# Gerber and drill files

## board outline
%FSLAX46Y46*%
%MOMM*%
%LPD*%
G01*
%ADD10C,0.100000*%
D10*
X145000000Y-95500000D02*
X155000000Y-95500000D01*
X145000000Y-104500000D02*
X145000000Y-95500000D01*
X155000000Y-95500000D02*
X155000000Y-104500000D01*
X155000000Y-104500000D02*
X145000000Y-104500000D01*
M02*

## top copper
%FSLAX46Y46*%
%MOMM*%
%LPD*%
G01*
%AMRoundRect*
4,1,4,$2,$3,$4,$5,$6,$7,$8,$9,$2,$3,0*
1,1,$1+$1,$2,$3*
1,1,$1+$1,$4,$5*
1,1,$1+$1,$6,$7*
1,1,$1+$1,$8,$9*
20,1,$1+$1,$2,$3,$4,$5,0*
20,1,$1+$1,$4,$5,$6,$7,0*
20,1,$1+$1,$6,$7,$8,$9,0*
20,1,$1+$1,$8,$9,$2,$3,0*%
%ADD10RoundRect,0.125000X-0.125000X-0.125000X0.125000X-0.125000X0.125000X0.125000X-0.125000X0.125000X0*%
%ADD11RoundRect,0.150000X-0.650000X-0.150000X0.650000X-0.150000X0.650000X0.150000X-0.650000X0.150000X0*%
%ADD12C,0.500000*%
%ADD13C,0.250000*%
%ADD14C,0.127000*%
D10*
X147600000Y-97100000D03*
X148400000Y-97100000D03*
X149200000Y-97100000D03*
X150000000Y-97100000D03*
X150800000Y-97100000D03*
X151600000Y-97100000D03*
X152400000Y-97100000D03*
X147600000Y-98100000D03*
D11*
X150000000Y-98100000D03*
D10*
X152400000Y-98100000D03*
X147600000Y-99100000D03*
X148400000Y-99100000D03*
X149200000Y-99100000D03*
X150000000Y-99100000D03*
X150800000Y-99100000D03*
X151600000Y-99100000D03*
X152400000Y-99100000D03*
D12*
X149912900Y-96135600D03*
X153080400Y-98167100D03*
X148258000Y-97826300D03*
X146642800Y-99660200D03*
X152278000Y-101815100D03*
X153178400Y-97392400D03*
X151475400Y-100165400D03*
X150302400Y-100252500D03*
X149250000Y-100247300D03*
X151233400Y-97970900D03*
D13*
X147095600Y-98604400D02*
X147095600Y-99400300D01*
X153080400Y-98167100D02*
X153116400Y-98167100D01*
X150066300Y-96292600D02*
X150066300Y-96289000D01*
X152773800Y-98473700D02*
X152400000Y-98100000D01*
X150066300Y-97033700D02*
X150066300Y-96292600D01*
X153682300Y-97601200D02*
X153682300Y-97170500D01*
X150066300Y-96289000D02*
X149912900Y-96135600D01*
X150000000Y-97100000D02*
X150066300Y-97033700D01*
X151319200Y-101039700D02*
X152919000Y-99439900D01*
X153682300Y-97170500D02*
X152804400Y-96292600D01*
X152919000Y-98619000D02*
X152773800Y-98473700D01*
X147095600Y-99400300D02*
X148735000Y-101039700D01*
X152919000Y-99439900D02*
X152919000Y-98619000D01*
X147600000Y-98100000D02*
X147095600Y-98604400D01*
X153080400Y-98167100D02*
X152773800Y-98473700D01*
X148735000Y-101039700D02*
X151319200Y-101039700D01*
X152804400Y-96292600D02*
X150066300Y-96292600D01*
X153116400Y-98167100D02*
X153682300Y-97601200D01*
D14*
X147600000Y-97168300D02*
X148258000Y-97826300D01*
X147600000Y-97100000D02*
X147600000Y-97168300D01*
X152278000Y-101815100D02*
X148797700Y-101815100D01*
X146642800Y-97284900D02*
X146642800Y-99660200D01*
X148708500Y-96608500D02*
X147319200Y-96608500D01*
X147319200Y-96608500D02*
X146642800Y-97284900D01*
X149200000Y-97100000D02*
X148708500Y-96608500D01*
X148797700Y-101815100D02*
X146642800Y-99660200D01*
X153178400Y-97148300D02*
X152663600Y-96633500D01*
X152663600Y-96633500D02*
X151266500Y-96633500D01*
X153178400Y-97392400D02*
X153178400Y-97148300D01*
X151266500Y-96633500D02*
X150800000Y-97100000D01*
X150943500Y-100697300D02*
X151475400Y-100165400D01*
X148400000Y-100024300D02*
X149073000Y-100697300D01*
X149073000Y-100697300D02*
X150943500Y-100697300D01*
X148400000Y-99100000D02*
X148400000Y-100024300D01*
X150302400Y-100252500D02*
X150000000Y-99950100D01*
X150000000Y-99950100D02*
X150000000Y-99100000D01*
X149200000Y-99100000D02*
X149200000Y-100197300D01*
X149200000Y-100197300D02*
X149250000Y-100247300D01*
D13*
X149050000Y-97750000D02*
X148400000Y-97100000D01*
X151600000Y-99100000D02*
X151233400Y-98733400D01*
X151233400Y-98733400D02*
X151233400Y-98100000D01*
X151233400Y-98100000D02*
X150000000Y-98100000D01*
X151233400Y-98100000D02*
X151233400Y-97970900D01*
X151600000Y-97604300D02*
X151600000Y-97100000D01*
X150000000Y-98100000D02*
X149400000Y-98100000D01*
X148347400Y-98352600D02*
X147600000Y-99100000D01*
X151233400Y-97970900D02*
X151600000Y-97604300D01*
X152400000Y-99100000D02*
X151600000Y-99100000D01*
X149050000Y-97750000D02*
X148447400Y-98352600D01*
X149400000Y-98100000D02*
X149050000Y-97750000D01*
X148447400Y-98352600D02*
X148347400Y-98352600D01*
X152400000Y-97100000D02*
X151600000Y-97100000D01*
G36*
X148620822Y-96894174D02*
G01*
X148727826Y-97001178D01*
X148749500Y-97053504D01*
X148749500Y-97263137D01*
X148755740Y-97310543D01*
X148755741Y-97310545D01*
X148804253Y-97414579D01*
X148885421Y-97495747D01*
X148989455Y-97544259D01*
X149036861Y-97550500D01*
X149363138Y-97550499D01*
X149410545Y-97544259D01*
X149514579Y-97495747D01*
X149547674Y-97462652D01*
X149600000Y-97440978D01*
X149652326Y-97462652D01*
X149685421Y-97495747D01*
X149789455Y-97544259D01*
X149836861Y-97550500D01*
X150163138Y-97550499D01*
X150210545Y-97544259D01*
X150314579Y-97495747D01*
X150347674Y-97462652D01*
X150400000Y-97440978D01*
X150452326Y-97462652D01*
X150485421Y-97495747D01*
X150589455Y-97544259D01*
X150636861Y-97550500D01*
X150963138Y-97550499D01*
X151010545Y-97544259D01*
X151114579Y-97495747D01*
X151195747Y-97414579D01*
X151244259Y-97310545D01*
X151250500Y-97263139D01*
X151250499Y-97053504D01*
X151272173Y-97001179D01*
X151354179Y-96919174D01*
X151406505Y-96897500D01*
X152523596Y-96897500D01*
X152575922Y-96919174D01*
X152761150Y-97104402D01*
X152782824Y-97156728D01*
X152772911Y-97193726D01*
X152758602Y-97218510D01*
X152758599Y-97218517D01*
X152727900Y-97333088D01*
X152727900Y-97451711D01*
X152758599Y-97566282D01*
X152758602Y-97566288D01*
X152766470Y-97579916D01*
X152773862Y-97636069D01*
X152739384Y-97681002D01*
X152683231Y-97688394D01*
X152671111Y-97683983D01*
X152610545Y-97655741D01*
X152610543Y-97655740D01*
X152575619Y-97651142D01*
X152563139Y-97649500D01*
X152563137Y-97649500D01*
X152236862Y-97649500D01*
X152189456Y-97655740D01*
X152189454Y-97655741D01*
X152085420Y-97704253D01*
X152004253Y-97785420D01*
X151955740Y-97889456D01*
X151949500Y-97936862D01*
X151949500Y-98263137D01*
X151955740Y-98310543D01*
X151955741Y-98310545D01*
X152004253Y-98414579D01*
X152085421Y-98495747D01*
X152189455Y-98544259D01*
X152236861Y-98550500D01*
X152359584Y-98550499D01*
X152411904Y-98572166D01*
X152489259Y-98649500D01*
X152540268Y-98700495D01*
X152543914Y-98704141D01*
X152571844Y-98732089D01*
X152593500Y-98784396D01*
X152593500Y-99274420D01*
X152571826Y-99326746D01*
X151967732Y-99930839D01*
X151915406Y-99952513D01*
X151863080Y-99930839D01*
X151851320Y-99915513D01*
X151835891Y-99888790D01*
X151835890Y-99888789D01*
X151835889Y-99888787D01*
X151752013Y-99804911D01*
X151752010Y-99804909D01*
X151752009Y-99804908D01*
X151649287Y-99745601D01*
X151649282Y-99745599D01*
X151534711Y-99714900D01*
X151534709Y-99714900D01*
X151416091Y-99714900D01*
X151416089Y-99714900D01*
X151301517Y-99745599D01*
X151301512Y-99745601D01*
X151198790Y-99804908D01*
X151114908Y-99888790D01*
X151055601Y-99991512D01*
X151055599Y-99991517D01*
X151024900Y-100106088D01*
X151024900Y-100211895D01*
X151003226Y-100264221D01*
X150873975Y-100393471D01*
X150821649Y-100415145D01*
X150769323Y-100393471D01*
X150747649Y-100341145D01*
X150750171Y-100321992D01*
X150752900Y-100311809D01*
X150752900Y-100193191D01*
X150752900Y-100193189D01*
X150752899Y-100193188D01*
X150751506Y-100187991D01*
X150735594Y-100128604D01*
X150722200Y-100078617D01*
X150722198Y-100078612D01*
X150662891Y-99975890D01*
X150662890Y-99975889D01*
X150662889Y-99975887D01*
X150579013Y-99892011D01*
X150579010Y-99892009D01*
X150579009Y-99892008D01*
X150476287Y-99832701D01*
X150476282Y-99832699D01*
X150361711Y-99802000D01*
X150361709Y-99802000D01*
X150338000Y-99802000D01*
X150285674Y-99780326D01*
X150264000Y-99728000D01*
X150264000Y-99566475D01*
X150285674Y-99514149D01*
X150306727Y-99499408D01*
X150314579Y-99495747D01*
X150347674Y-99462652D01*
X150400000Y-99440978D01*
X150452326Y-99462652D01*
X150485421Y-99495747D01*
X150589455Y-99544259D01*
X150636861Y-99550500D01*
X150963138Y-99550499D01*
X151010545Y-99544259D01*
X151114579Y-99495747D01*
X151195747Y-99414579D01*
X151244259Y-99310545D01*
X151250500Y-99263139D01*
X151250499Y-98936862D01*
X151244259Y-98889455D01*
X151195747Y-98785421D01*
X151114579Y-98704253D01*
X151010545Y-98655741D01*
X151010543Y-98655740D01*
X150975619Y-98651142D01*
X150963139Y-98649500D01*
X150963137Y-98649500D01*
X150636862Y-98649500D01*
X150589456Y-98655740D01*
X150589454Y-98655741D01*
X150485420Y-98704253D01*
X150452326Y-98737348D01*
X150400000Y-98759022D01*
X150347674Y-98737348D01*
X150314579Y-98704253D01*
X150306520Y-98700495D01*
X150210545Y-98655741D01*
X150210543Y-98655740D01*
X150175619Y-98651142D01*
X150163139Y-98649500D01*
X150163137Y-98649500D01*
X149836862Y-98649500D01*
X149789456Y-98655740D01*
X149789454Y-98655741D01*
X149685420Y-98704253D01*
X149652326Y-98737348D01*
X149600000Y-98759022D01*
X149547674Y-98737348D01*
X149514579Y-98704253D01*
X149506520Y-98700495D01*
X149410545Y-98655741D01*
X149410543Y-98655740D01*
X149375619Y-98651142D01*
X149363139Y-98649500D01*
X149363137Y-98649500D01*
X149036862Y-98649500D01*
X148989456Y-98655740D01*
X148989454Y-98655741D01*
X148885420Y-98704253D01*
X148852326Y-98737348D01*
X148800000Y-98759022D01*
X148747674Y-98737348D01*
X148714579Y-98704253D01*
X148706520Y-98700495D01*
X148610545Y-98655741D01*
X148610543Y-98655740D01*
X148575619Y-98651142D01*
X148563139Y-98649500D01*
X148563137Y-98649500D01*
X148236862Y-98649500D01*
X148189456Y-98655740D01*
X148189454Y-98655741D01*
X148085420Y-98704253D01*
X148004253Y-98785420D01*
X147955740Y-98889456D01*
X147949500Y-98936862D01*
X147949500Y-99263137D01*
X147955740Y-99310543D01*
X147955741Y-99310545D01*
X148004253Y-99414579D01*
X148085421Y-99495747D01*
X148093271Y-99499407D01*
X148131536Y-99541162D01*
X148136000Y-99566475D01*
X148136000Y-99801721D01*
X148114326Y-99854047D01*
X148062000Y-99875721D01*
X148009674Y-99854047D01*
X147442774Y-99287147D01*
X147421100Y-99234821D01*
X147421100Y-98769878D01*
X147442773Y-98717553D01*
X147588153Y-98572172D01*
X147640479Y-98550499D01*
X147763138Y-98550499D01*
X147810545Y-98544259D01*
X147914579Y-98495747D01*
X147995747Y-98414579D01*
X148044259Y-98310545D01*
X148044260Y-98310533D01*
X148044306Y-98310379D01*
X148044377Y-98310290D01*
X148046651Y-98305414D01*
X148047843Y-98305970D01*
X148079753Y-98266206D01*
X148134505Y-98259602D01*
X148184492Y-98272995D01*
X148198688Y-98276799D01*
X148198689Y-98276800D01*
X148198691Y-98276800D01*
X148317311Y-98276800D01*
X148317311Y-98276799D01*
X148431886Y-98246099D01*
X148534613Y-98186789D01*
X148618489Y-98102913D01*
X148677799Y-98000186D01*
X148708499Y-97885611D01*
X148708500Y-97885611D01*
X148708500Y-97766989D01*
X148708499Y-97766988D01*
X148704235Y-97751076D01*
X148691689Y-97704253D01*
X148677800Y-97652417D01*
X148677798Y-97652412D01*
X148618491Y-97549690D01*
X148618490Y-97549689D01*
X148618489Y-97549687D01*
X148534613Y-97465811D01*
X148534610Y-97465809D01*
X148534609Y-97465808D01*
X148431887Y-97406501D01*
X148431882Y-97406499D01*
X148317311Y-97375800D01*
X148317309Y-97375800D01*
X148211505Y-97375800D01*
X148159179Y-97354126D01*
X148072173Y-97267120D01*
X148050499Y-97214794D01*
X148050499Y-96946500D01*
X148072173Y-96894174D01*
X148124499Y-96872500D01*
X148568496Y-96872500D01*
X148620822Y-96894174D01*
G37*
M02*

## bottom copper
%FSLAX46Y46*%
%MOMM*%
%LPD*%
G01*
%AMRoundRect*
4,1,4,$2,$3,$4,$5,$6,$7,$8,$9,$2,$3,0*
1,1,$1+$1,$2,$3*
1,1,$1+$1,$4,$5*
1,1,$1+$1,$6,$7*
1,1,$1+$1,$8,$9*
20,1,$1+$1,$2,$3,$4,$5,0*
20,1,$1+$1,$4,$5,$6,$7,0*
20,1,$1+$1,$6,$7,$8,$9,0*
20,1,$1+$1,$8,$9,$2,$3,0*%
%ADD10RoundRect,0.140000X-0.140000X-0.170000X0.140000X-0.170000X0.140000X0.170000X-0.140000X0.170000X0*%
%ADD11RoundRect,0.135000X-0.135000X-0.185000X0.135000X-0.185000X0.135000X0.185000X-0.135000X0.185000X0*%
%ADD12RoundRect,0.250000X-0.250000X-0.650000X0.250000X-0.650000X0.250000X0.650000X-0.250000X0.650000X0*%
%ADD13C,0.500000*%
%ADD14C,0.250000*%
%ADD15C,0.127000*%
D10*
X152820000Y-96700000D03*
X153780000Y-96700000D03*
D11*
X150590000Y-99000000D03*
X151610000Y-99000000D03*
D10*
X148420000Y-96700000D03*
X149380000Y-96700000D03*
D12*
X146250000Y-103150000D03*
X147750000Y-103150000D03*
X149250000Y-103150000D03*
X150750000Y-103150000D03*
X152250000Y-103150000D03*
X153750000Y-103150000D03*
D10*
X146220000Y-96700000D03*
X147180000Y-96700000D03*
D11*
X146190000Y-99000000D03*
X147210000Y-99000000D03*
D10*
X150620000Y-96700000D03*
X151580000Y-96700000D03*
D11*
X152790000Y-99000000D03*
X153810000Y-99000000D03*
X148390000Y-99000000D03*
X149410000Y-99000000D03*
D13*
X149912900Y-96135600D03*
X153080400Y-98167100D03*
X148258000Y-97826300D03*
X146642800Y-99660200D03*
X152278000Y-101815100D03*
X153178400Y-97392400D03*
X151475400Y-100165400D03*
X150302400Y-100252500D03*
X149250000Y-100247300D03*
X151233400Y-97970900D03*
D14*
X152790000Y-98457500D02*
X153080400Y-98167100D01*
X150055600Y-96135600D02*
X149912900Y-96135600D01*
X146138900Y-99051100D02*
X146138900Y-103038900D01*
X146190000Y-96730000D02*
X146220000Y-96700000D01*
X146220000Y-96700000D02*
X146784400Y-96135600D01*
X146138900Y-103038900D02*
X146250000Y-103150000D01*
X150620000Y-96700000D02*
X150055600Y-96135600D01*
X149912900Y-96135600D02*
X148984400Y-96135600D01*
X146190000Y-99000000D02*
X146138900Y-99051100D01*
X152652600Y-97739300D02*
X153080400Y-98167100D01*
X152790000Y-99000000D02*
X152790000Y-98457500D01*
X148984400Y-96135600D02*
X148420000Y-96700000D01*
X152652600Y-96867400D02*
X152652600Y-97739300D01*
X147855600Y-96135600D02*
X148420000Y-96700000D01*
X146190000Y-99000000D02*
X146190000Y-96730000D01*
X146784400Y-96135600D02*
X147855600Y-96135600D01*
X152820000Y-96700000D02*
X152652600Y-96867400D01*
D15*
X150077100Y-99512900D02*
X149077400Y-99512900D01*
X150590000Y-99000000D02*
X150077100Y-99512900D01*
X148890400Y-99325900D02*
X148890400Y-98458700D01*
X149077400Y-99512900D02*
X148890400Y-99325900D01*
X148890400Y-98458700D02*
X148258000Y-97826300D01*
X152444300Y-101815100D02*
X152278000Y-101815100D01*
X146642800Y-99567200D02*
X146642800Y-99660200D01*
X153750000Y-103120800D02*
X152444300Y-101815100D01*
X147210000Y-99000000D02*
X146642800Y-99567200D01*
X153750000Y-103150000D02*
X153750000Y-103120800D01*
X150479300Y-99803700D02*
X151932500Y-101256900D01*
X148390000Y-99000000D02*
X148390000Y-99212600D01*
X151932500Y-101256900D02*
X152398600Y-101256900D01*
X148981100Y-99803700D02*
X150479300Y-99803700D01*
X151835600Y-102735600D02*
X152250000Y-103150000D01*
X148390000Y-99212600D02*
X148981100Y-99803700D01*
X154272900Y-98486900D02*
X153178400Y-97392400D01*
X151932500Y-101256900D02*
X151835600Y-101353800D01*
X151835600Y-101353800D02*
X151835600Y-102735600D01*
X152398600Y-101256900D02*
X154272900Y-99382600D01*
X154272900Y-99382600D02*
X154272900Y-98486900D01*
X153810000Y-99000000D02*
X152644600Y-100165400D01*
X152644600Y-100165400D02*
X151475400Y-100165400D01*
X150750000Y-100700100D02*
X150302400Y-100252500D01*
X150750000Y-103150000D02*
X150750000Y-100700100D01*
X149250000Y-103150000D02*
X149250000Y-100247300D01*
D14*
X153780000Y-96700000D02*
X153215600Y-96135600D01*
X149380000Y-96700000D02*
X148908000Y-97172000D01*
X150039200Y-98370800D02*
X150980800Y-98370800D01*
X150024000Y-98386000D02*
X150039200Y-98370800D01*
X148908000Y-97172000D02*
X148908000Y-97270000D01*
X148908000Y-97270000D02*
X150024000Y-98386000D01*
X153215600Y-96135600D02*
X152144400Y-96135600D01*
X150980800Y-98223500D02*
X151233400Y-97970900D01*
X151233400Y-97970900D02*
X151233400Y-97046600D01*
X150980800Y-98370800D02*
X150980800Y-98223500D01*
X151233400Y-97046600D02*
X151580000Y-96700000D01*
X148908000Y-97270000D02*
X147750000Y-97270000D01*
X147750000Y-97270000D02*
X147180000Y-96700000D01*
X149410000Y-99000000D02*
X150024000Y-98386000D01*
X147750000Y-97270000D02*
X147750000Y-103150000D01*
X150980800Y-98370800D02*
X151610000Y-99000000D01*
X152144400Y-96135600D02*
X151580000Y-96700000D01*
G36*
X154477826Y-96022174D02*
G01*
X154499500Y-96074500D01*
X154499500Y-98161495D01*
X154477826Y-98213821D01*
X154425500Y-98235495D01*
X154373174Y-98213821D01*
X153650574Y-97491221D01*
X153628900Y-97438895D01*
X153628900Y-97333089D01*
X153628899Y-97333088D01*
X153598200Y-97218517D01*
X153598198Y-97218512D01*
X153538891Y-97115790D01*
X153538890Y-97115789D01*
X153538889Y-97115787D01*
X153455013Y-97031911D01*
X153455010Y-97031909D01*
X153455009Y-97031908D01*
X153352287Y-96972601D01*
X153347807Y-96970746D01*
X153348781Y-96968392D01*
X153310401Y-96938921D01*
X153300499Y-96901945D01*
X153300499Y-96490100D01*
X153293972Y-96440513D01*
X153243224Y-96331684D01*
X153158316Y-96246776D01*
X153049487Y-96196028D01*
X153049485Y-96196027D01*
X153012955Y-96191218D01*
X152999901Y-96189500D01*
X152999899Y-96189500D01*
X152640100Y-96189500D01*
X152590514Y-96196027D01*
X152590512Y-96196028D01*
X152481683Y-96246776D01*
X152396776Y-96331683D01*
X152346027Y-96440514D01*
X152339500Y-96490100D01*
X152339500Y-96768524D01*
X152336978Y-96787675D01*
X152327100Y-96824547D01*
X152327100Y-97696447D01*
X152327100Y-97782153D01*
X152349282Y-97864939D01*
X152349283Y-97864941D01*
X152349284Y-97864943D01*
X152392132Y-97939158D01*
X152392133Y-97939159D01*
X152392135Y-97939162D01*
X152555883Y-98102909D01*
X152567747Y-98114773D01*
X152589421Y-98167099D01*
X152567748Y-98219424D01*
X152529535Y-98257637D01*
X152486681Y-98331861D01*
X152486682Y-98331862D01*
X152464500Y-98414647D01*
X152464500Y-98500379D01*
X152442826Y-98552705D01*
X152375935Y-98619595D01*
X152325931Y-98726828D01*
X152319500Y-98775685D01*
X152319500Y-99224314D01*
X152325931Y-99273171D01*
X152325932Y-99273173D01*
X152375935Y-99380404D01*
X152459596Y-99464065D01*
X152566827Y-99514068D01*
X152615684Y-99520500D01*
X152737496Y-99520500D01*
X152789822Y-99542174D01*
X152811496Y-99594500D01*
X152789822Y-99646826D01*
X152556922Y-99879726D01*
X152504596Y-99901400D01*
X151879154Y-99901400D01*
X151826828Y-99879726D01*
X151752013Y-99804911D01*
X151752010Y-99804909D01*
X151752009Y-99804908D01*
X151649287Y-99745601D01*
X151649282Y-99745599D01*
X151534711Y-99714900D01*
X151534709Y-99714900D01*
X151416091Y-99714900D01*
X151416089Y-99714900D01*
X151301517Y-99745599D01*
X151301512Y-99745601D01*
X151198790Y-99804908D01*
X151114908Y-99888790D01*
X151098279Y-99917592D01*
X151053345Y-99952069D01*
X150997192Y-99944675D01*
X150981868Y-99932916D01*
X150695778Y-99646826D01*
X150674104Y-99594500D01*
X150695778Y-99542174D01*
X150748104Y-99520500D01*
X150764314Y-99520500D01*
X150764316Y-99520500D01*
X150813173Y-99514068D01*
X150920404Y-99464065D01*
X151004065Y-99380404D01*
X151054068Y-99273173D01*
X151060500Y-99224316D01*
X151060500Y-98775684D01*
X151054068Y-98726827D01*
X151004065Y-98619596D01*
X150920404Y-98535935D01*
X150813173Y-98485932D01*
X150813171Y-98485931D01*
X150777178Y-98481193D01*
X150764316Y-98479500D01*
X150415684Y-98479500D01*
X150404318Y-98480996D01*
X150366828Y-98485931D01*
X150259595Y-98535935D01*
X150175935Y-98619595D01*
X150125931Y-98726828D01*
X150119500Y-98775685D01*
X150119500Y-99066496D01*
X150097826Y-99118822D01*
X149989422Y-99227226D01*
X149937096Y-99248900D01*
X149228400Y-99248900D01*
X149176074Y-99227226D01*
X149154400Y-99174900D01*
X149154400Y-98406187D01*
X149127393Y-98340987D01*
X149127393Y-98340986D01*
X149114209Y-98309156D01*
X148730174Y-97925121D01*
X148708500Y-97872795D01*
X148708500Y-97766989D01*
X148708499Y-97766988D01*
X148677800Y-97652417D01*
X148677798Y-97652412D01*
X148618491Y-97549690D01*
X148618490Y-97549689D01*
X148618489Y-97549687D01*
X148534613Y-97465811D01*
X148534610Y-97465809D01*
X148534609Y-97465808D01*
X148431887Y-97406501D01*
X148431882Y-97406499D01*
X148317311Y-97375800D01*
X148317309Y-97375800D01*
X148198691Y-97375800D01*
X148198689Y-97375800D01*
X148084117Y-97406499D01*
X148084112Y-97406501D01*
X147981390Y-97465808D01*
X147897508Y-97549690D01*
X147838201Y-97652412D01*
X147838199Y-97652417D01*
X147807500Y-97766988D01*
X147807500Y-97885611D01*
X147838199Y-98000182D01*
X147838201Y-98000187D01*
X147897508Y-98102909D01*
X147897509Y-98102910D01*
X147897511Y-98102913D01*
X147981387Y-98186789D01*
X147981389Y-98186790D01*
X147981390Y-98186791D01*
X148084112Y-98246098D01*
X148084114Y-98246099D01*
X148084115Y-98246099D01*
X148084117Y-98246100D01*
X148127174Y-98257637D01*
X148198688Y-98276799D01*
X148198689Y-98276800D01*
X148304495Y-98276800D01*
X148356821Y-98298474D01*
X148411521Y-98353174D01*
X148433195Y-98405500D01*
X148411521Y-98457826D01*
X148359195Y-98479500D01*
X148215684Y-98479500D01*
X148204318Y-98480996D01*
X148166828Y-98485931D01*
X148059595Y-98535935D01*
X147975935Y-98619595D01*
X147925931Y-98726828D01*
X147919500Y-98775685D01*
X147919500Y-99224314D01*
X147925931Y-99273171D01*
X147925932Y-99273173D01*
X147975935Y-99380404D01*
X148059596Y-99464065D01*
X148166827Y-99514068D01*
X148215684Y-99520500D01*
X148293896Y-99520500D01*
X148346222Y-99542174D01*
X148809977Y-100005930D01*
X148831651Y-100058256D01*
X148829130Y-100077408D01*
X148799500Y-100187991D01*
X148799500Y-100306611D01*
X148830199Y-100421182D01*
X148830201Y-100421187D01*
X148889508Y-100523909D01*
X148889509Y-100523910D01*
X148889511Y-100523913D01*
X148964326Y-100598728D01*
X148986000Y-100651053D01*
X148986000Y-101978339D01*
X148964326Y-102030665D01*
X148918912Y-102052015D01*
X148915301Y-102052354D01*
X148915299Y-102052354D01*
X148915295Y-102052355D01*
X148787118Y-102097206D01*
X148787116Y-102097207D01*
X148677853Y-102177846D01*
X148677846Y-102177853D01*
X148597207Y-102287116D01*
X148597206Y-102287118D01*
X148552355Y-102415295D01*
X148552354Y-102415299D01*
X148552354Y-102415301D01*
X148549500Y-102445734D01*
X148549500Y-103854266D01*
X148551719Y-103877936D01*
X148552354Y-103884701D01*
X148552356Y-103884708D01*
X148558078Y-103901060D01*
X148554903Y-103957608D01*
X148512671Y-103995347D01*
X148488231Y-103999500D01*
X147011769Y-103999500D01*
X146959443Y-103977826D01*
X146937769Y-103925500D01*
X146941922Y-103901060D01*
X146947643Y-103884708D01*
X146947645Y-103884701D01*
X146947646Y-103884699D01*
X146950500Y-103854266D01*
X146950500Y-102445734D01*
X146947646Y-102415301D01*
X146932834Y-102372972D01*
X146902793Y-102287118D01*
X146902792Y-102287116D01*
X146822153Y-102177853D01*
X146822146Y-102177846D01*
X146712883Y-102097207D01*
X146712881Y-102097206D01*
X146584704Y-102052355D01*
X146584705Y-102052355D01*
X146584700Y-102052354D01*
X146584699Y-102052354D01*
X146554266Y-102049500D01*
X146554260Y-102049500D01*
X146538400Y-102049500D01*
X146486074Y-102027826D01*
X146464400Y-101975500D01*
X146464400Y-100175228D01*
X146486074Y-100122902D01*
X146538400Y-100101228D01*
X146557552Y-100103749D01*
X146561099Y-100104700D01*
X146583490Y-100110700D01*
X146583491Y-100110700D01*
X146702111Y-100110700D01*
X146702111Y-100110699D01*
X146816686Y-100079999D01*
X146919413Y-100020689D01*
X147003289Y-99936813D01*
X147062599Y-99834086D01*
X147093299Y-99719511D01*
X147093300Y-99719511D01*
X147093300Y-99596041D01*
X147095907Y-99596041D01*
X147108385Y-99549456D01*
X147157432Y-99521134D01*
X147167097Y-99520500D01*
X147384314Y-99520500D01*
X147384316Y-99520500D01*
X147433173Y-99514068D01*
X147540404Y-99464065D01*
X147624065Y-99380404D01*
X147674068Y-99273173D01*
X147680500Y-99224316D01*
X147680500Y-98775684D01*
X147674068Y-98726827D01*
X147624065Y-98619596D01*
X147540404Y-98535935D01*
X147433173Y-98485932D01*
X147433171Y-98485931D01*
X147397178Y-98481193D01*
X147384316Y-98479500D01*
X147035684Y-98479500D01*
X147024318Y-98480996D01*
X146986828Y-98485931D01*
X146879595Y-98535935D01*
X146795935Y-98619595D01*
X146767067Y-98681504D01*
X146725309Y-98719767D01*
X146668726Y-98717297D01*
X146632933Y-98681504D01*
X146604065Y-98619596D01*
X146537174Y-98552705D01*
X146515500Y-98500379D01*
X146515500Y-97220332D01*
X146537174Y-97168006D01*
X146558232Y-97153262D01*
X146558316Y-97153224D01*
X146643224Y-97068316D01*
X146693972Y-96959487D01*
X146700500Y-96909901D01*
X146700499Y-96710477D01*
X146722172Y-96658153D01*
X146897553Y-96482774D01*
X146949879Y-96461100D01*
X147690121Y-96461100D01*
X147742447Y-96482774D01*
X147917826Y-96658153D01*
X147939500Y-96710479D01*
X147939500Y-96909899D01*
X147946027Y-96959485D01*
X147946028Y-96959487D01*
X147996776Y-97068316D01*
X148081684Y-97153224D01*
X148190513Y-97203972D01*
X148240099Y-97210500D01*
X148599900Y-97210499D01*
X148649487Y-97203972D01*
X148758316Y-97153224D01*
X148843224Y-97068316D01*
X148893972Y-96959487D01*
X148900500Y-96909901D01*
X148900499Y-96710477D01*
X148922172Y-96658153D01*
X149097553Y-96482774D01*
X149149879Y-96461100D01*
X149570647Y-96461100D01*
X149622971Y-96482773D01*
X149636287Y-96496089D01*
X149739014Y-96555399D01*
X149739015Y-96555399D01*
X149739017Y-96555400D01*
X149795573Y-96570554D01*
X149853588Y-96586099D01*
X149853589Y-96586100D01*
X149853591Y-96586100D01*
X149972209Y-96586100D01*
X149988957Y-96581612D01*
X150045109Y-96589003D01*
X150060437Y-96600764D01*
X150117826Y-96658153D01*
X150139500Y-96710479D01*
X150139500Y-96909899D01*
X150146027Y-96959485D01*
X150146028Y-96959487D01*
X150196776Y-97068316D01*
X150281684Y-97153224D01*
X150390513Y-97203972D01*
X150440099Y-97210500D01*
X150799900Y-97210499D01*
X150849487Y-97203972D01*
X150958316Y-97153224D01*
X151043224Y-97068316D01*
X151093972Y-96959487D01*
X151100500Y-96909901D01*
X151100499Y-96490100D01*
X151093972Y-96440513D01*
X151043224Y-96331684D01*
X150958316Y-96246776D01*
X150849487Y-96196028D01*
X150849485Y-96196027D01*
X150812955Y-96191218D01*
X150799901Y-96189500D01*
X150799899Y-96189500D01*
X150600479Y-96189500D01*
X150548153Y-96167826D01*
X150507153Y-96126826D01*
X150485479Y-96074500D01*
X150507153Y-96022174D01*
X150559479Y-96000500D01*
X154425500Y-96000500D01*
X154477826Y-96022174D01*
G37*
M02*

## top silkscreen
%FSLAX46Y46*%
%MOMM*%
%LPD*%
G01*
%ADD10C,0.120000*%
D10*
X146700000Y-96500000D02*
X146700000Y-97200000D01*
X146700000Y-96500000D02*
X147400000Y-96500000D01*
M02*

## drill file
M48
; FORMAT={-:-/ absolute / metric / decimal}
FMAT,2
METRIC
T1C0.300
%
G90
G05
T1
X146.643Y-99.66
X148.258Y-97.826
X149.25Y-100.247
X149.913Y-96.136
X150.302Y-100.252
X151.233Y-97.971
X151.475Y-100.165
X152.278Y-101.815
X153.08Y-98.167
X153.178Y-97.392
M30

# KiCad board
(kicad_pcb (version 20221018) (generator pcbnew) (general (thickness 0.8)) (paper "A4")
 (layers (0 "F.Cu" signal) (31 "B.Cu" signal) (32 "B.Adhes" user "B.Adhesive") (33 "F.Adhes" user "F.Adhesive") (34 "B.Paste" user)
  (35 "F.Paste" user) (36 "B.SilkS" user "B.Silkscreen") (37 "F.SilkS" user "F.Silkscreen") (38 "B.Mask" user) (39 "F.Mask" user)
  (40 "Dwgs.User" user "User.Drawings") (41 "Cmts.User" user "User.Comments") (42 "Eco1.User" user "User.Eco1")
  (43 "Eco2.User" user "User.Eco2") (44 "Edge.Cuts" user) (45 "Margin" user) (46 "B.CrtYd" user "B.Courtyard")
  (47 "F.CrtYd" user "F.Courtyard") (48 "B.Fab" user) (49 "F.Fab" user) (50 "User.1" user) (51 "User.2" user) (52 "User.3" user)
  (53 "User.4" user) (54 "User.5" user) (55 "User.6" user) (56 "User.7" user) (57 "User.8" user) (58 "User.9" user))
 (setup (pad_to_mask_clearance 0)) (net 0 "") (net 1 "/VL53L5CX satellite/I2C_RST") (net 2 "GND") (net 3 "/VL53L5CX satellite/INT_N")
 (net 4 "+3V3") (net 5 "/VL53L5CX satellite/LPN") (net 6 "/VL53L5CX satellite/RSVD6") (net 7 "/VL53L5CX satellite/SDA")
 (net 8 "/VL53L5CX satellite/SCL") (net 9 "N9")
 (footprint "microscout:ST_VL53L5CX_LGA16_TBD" (layer "F.Cu") (at 150 98.1)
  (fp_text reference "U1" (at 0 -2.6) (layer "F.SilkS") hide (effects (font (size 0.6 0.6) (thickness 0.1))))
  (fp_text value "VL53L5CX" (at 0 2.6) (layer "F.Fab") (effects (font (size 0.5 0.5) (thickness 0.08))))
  (fp_line (start -3.3 -1.6) (end -3.3 -0.9) (stroke (width 0.12) (type solid)) (layer "F.SilkS"))
  (fp_line (start -3.3 -1.6) (end -2.6 -1.6) (stroke (width 0.12) (type solid)) (layer "F.SilkS"))
  (pad "A1" smd roundrect (at -2.4 -1) (size 0.5 0.5) (layers "F.Cu" "F.Paste" "F.Mask") (roundrect_rratio 0.25)
   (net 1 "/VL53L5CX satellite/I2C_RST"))
  (pad "A2" smd roundrect (at -1.6 -1) (size 0.5 0.5) (layers "F.Cu" "F.Paste" "F.Mask") (roundrect_rratio 0.25) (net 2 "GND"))
  (pad "A3" smd roundrect (at -0.8 -1) (size 0.5 0.5) (layers "F.Cu" "F.Paste" "F.Mask") (roundrect_rratio 0.25)
   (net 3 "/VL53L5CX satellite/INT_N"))
  (pad "A4" smd roundrect (at 0 -1) (size 0.5 0.5) (layers "F.Cu" "F.Paste" "F.Mask") (roundrect_rratio 0.25) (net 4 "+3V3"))
  (pad "A5" smd roundrect (at 0.8 -1) (size 0.5 0.5) (layers "F.Cu" "F.Paste" "F.Mask") (roundrect_rratio 0.25)
   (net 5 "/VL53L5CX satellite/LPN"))
  (pad "A6" smd roundrect (at 1.6 -1) (size 0.5 0.5) (layers "F.Cu" "F.Paste" "F.Mask") (roundrect_rratio 0.25) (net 2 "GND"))
  (pad "A7" smd roundrect (at 2.4 -1) (size 0.5 0.5) (layers "F.Cu" "F.Paste" "F.Mask") (roundrect_rratio 0.25) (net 2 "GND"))
  (pad "B1" smd roundrect (at -2.4 0) (size 0.5 0.5) (layers "F.Cu" "F.Paste" "F.Mask") (roundrect_rratio 0.25) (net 4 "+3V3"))
  (pad "B4" smd roundrect (at 0 0) (size 1.6 0.6) (layers "F.Cu" "F.Paste" "F.Mask") (roundrect_rratio 0.25) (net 2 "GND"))
  (pad "B7" smd roundrect (at 2.4 0) (size 0.5 0.5) (layers "F.Cu" "F.Paste" "F.Mask") (roundrect_rratio 0.25) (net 4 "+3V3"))
  (pad "C1" smd roundrect (at -2.4 1) (size 0.5 0.5) (layers "F.Cu" "F.Paste" "F.Mask") (roundrect_rratio 0.25) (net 2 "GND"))
  (pad "C2" smd roundrect (at -1.6 1) (size 0.5 0.5) (layers "F.Cu" "F.Paste" "F.Mask") (roundrect_rratio 0.25)
   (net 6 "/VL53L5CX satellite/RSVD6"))
  (pad "C3" smd roundrect (at -0.8 1) (size 0.5 0.5) (layers "F.Cu" "F.Paste" "F.Mask") (roundrect_rratio 0.25)
   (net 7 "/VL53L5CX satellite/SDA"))
  (pad "C4" smd roundrect (at 0 1) (size 0.5 0.5) (layers "F.Cu" "F.Paste" "F.Mask") (roundrect_rratio 0.25)
   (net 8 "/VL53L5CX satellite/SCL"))
  (pad "C5" smd roundrect (at 0.8 1) (size 0.5 0.5) (layers "F.Cu" "F.Paste" "F.Mask") (roundrect_rratio 0.25) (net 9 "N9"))
  (pad "C6" smd roundrect (at 1.6 1) (size 0.5 0.5) (layers "F.Cu" "F.Paste" "F.Mask") (roundrect_rratio 0.25) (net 2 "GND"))
  (pad "C7" smd roundrect (at 2.4 1) (size 0.5 0.5) (layers "F.Cu" "F.Paste" "F.Mask") (roundrect_rratio 0.25) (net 2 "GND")))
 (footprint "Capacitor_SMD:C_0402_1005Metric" (layer "B.Cu") (at 153.3 96.7)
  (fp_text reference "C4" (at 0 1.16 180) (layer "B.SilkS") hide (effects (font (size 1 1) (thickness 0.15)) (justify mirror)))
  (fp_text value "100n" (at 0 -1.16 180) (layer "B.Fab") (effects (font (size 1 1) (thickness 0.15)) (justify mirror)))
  (pad "1" smd roundrect (at -0.48 0) (size 0.56 0.62) (layers "B.Cu" "B.Paste" "B.Mask") (roundrect_rratio 0.25) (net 4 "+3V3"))
  (pad "2" smd roundrect (at 0.48 0) (size 0.56 0.62) (layers "B.Cu" "B.Paste" "B.Mask") (roundrect_rratio 0.25) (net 2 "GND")))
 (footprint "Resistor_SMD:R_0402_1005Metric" (layer "B.Cu") (at 151.1 99)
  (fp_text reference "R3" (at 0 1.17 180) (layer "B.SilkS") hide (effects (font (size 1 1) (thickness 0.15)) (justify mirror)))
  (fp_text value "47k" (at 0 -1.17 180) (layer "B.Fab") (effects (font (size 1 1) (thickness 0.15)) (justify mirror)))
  (pad "1" smd roundrect (at -0.51 0) (size 0.54 0.64) (layers "B.Cu" "B.Paste" "B.Mask") (roundrect_rratio 0.25)
   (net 1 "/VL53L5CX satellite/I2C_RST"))
  (pad "2" smd roundrect (at 0.51 0) (size 0.54 0.64) (layers "B.Cu" "B.Paste" "B.Mask") (roundrect_rratio 0.25) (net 2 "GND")))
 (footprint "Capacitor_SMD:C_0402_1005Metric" (layer "B.Cu") (at 148.9 96.7)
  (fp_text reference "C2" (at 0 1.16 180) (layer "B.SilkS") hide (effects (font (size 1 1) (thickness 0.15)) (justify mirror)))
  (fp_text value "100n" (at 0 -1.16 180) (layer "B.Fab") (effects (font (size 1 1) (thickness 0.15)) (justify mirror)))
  (pad "1" smd roundrect (at -0.48 0) (size 0.56 0.62) (layers "B.Cu" "B.Paste" "B.Mask") (roundrect_rratio 0.25) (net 4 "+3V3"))
  (pad "2" smd roundrect (at 0.48 0) (size 0.56 0.62) (layers "B.Cu" "B.Paste" "B.Mask") (roundrect_rratio 0.25) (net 2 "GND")))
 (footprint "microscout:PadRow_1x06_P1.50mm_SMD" (layer "B.Cu") (at 150 103.15)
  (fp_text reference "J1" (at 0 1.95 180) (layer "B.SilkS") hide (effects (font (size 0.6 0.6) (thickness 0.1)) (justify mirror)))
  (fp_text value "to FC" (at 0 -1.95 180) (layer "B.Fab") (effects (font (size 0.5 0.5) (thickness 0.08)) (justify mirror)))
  (pad "1" smd roundrect (at -3.75 0) (size 1 1.8) (layers "B.Cu" "B.Paste" "B.Mask") (roundrect_rratio 0.25) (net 4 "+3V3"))
  (pad "2" smd roundrect (at -2.25 0) (size 1 1.8) (layers "B.Cu" "B.Paste" "B.Mask") (roundrect_rratio 0.25) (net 2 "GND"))
  (pad "3" smd roundrect (at -0.75 0) (size 1 1.8) (layers "B.Cu" "B.Paste" "B.Mask") (roundrect_rratio 0.25)
   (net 7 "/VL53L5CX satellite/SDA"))
  (pad "4" smd roundrect (at 0.75 0) (size 1 1.8) (layers "B.Cu" "B.Paste" "B.Mask") (roundrect_rratio 0.25)
   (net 8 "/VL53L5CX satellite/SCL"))
  (pad "5" smd roundrect (at 2.25 0) (size 1 1.8) (layers "B.Cu" "B.Paste" "B.Mask") (roundrect_rratio 0.25)
   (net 5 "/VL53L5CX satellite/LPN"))
  (pad "6" smd roundrect (at 3.75 0) (size 1 1.8) (layers "B.Cu" "B.Paste" "B.Mask") (roundrect_rratio 0.25)
   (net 3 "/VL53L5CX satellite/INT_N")))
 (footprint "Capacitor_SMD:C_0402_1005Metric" (layer "B.Cu") (at 146.7 96.7)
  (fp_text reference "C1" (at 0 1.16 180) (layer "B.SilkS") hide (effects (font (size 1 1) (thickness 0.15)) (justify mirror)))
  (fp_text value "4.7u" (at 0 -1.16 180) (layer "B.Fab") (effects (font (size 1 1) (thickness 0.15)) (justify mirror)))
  (pad "1" smd roundrect (at -0.48 0) (size 0.56 0.62) (layers "B.Cu" "B.Paste" "B.Mask") (roundrect_rratio 0.25) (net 4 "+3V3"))
  (pad "2" smd roundrect (at 0.48 0) (size 0.56 0.62) (layers "B.Cu" "B.Paste" "B.Mask") (roundrect_rratio 0.25) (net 2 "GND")))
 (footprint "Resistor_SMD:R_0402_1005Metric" (layer "B.Cu") (at 146.7 99)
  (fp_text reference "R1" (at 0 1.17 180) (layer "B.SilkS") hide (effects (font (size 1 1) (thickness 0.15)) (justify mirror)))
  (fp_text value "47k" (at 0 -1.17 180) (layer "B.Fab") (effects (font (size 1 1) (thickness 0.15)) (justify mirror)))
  (pad "1" smd roundrect (at -0.51 0) (size 0.54 0.64) (layers "B.Cu" "B.Paste" "B.Mask") (roundrect_rratio 0.25) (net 4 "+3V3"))
  (pad "2" smd roundrect (at 0.51 0) (size 0.54 0.64) (layers "B.Cu" "B.Paste" "B.Mask") (roundrect_rratio 0.25)
   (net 3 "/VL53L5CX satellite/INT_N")))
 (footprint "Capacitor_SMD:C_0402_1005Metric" (layer "B.Cu") (at 151.1 96.7)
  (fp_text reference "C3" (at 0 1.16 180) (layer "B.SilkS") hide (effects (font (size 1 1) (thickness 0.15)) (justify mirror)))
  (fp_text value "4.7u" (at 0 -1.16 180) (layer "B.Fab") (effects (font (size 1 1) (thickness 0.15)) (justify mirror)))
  (pad "1" smd roundrect (at -0.48 0) (size 0.56 0.62) (layers "B.Cu" "B.Paste" "B.Mask") (roundrect_rratio 0.25) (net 4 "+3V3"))
  (pad "2" smd roundrect (at 0.48 0) (size 0.56 0.62) (layers "B.Cu" "B.Paste" "B.Mask") (roundrect_rratio 0.25) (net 2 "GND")))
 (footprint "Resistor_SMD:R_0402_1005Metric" (layer "B.Cu") (at 153.3 99)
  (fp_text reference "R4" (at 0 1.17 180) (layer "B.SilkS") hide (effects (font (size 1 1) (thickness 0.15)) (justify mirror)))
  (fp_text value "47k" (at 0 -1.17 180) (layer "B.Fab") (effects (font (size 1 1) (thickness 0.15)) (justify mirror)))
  (pad "1" smd roundrect (at -0.51 0) (size 0.54 0.64) (layers "B.Cu" "B.Paste" "B.Mask") (roundrect_rratio 0.25) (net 4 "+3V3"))
  (pad "2" smd roundrect (at 0.51 0) (size 0.54 0.64) (layers "B.Cu" "B.Paste" "B.Mask") (roundrect_rratio 0.25)
   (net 6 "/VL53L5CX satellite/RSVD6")))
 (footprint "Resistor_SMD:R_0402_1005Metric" (layer "B.Cu") (at 148.9 99)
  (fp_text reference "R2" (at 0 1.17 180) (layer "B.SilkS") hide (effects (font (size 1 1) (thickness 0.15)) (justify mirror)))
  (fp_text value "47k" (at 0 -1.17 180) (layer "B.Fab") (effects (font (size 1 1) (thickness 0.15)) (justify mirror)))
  (pad "1" smd roundrect (at -0.51 0) (size 0.54 0.64) (layers "B.Cu" "B.Paste" "B.Mask") (roundrect_rratio 0.25)
   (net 5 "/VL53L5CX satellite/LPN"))
  (pad "2" smd roundrect (at 0.51 0) (size 0.54 0.64) (layers "B.Cu" "B.Paste" "B.Mask") (roundrect_rratio 0.25) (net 2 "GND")))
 (gr_line (start 145 95.5) (end 155 95.5) (stroke (width 0.1) (type default)) (layer "Edge.Cuts"))
 (gr_line (start 145 104.5) (end 145 95.5) (stroke (width 0.1) (type default)) (layer "Edge.Cuts"))
 (gr_line (start 155 95.5) (end 155 104.5) (stroke (width 0.1) (type default)) (layer "Edge.Cuts"))
 (gr_line (start 155 104.5) (end 145 104.5) (stroke (width 0.1) (type default)) (layer "Edge.Cuts"))
 (segment (start 147.0956 98.6044) (end 147.0956 99.4003) (width 0.25) (layer "F.Cu") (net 4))
 (segment (start 153.0804 98.1671) (end 153.1164 98.1671) (width 0.25) (layer "F.Cu") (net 4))
 (segment (start 150.0663 96.2926) (end 150.0663 96.289) (width 0.25) (layer "F.Cu") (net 4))
 (segment (start 152.7738 98.4737) (end 152.4 98.1) (width 0.25) (layer "F.Cu") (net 4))
 (segment (start 150.0663 97.0337) (end 150.0663 96.2926) (width 0.25) (layer "F.Cu") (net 4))
 (segment (start 153.6823 97.6012) (end 153.6823 97.1705) (width 0.25) (layer "F.Cu") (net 4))
 (segment (start 150.0663 96.289) (end 149.9129 96.1356) (width 0.25) (layer "F.Cu") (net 4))
 (segment (start 150 97.1) (end 150.0663 97.0337) (width 0.25) (layer "F.Cu") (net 4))
 (segment (start 151.3192 101.0397) (end 152.919 99.4399) (width 0.25) (layer "F.Cu") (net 4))
 (segment (start 153.6823 97.1705) (end 152.8044 96.2926) (width 0.25) (layer "F.Cu") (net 4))
 (segment (start 152.919 98.619) (end 152.7738 98.4737) (width 0.25) (layer "F.Cu") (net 4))
 (segment (start 147.0956 99.4003) (end 148.735 101.0397) (width 0.25) (layer "F.Cu") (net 4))
 (segment (start 152.919 99.4399) (end 152.919 98.619) (width 0.25) (layer "F.Cu") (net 4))
 (segment (start 147.6 98.1) (end 147.0956 98.6044) (width 0.25) (layer "F.Cu") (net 4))
 (segment (start 153.0804 98.1671) (end 152.7738 98.4737) (width 0.25) (layer "F.Cu") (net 4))
 (segment (start 148.735 101.0397) (end 151.3192 101.0397) (width 0.25) (layer "F.Cu") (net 4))
 (segment (start 152.8044 96.2926) (end 150.0663 96.2926) (width 0.25) (layer "F.Cu") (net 4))
 (segment (start 153.1164 98.1671) (end 153.6823 97.6012) (width 0.25) (layer "F.Cu") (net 4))
 (via (at 149.9129 96.1356) (size 0.5) (drill 0.3) (layers "F.Cu" "B.Cu") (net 4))
 (via (at 153.0804 98.1671) (size 0.5) (drill 0.3) (layers "F.Cu" "B.Cu") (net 4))
 (segment (start 152.79 98.4575) (end 153.0804 98.1671) (width 0.25) (layer "B.Cu") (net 4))
 (segment (start 150.0556 96.1356) (end 149.9129 96.1356) (width 0.25) (layer "B.Cu") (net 4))
 (segment (start 146.1389 99.0511) (end 146.1389 103.0389) (width 0.25) (layer "B.Cu") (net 4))
 (segment (start 146.19 96.73) (end 146.22 96.7) (width 0.25) (layer "B.Cu") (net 4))
 (segment (start 146.22 96.7) (end 146.7844 96.1356) (width 0.25) (layer "B.Cu") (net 4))
 (segment (start 146.1389 103.0389) (end 146.25 103.15) (width 0.25) (layer "B.Cu") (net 4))
 (segment (start 150.62 96.7) (end 150.0556 96.1356) (width 0.25) (layer "B.Cu") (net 4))
 (segment (start 149.9129 96.1356) (end 148.9844 96.1356) (width 0.25) (layer "B.Cu") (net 4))
 (segment (start 146.19 99) (end 146.1389 99.0511) (width 0.25) (layer "B.Cu") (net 4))
 (segment (start 152.6526 97.7393) (end 153.0804 98.1671) (width 0.25) (layer "B.Cu") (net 4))
 (segment (start 152.79 99) (end 152.79 98.4575) (width 0.25) (layer "B.Cu") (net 4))
 (segment (start 148.9844 96.1356) (end 148.42 96.7) (width 0.25) (layer "B.Cu") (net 4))
 (segment (start 152.6526 96.8674) (end 152.6526 97.7393) (width 0.25) (layer "B.Cu") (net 4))
 (segment (start 147.8556 96.1356) (end 148.42 96.7) (width 0.25) (layer "B.Cu") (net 4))
 (segment (start 146.19 99) (end 146.19 96.73) (width 0.25) (layer "B.Cu") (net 4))
 (segment (start 146.7844 96.1356) (end 147.8556 96.1356) (width 0.25) (layer "B.Cu") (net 4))
 (segment (start 152.82 96.7) (end 152.6526 96.8674) (width 0.25) (layer "B.Cu") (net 4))
 (segment (start 147.6 97.1683) (end 148.258 97.8263) (width 0.127) (layer "F.Cu") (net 1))
 (segment (start 147.6 97.1) (end 147.6 97.1683) (width 0.127) (layer "F.Cu") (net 1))
 (via (at 148.258 97.8263) (size 0.5) (drill 0.3) (layers "F.Cu" "B.Cu") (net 1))
 (segment (start 150.0771 99.5129) (end 149.0774 99.5129) (width 0.127) (layer "B.Cu") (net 1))
 (segment (start 150.59 99) (end 150.0771 99.5129) (width 0.127) (layer "B.Cu") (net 1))
 (segment (start 148.8904 99.3259) (end 148.8904 98.4587) (width 0.127) (layer "B.Cu") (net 1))
 (segment (start 149.0774 99.5129) (end 148.8904 99.3259) (width 0.127) (layer "B.Cu") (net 1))
 (segment (start 148.8904 98.4587) (end 148.258 97.8263) (width 0.127) (layer "B.Cu") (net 1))
 (segment (start 152.278 101.8151) (end 148.7977 101.8151) (width 0.127) (layer "F.Cu") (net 3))
 (segment (start 146.6428 97.2849) (end 146.6428 99.6602) (width 0.127) (layer "F.Cu") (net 3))
 (segment (start 148.7085 96.6085) (end 147.3192 96.6085) (width 0.127) (layer "F.Cu") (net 3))
 (segment (start 147.3192 96.6085) (end 146.6428 97.2849) (width 0.127) (layer "F.Cu") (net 3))
 (segment (start 149.2 97.1) (end 148.7085 96.6085) (width 0.127) (layer "F.Cu") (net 3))
 (segment (start 148.7977 101.8151) (end 146.6428 99.6602) (width 0.127) (layer "F.Cu") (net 3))
 (via (at 146.6428 99.6602) (size 0.5) (drill 0.3) (layers "F.Cu" "B.Cu") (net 3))
 (via (at 152.278 101.8151) (size 0.5) (drill 0.3) (layers "F.Cu" "B.Cu") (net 3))
 (segment (start 152.4443 101.8151) (end 152.278 101.8151) (width 0.127) (layer "B.Cu") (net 3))
 (segment (start 146.6428 99.5672) (end 146.6428 99.6602) (width 0.127) (layer "B.Cu") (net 3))
 (segment (start 153.75 103.1208) (end 152.4443 101.8151) (width 0.127) (layer "B.Cu") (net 3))
 (segment (start 147.21 99) (end 146.6428 99.5672) (width 0.127) (layer "B.Cu") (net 3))
 (segment (start 153.75 103.15) (end 153.75 103.1208) (width 0.127) (layer "B.Cu") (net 3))
 (segment (start 153.1784 97.1483) (end 152.6636 96.6335) (width 0.127) (layer "F.Cu") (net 5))
 (segment (start 152.6636 96.6335) (end 151.2665 96.6335) (width 0.127) (layer "F.Cu") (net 5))
 (segment (start 153.1784 97.3924) (end 153.1784 97.1483) (width 0.127) (layer "F.Cu") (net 5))
 (segment (start 151.2665 96.6335) (end 150.8 97.1) (width 0.127) (layer "F.Cu") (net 5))
 (via (at 153.1784 97.3924) (size 0.5) (drill 0.3) (layers "F.Cu" "B.Cu") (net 5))
 (segment (start 150.4793 99.8037) (end 151.9325 101.2569) (width 0.127) (layer "B.Cu") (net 5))
 (segment (start 148.39 99) (end 148.39 99.2126) (width 0.127) (layer "B.Cu") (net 5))
 (segment (start 151.9325 101.2569) (end 152.3986 101.2569) (width 0.127) (layer "B.Cu") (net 5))
 (segment (start 148.9811 99.8037) (end 150.4793 99.8037) (width 0.127) (layer "B.Cu") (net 5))
 (segment (start 151.8356 102.7356) (end 152.25 103.15) (width 0.127) (layer "B.Cu") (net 5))
 (segment (start 148.39 99.2126) (end 148.9811 99.8037) (width 0.127) (layer "B.Cu") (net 5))
 (segment (start 154.2729 98.4869) (end 153.1784 97.3924) (width 0.127) (layer "B.Cu") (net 5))
 (segment (start 151.9325 101.2569) (end 151.8356 101.3538) (width 0.127) (layer "B.Cu") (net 5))
 (segment (start 151.8356 101.3538) (end 151.8356 102.7356) (width 0.127) (layer "B.Cu") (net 5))
 (segment (start 152.3986 101.2569) (end 154.2729 99.3826) (width 0.127) (layer "B.Cu") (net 5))
 (segment (start 154.2729 99.3826) (end 154.2729 98.4869) (width 0.127) (layer "B.Cu") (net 5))
 (segment (start 150.9435 100.6973) (end 151.4754 100.1654) (width 0.127) (layer "F.Cu") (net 6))
 (segment (start 148.4 100.0243) (end 149.073 100.6973) (width 0.127) (layer "F.Cu") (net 6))
 (segment (start 149.073 100.6973) (end 150.9435 100.6973) (width 0.127) (layer "F.Cu") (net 6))
 (segment (start 148.4 99.1) (end 148.4 100.0243) (width 0.127) (layer "F.Cu") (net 6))
 (via (at 151.4754 100.1654) (size 0.5) (drill 0.3) (layers "F.Cu" "B.Cu") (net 6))
 (segment (start 153.81 99) (end 152.6446 100.1654) (width 0.127) (layer "B.Cu") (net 6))
 (segment (start 152.6446 100.1654) (end 151.4754 100.1654) (width 0.127) (layer "B.Cu") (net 6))
 (segment (start 150.3024 100.2525) (end 150 99.9501) (width 0.127) (layer "F.Cu") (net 8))
 (segment (start 150 99.9501) (end 150 99.1) (width 0.127) (layer "F.Cu") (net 8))
 (via (at 150.3024 100.2525) (size 0.5) (drill 0.3) (layers "F.Cu" "B.Cu") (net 8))
 (segment (start 150.75 100.7001) (end 150.3024 100.2525) (width 0.127) (layer "B.Cu") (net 8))
 (segment (start 150.75 103.15) (end 150.75 100.7001) (width 0.127) (layer "B.Cu") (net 8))
 (segment (start 149.2 99.1) (end 149.2 100.1973) (width 0.127) (layer "F.Cu") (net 7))
 (segment (start 149.2 100.1973) (end 149.25 100.2473) (width 0.127) (layer "F.Cu") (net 7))
 (via (at 149.25 100.2473) (size 0.5) (drill 0.3) (layers "F.Cu" "B.Cu") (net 7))
 (segment (start 149.25 103.15) (end 149.25 100.2473) (width 0.127) (layer "B.Cu") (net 7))
 (segment (start 149.05 97.75) (end 148.4 97.1) (width 0.25) (layer "F.Cu") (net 2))
 (segment (start 151.6 99.1) (end 151.2334 98.7334) (width 0.25) (layer "F.Cu") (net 2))
 (segment (start 151.2334 98.7334) (end 151.2334 98.1) (width 0.25) (layer "F.Cu") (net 2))
 (segment (start 151.2334 98.1) (end 150 98.1) (width 0.25) (layer "F.Cu") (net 2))
 (segment (start 151.2334 98.1) (end 151.2334 97.9709) (width 0.25) (layer "F.Cu") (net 2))
 (segment (start 151.6 97.6043) (end 151.6 97.1) (width 0.25) (layer "F.Cu") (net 2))
 (segment (start 150 98.1) (end 149.4 98.1) (width 0.25) (layer "F.Cu") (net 2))
 (segment (start 148.3474 98.3526) (end 147.6 99.1) (width 0.25) (layer "F.Cu") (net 2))
 (segment (start 151.2334 97.9709) (end 151.6 97.6043) (width 0.25) (layer "F.Cu") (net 2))
 (segment (start 152.4 99.1) (end 151.6 99.1) (width 0.25) (layer "F.Cu") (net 2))
 (segment (start 149.05 97.75) (end 148.4474 98.3526) (width 0.25) (layer "F.Cu") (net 2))
 (segment (start 149.4 98.1) (end 149.05 97.75) (width 0.25) (layer "F.Cu") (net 2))
 (segment (start 148.4474 98.3526) (end 148.3474 98.3526) (width 0.25) (layer "F.Cu") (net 2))
 (segment (start 152.4 97.1) (end 151.6 97.1) (width 0.25) (layer "F.Cu") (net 2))
 (via (at 151.2334 97.9709) (size 0.5) (drill 0.3) (layers "F.Cu" "B.Cu") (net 2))
 (segment (start 153.78 96.7) (end 153.2156 96.1356) (width 0.25) (layer "B.Cu") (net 2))
 (segment (start 149.38 96.7) (end 148.908 97.172) (width 0.25) (layer "B.Cu") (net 2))
 (segment (start 150.0392 98.3708) (end 150.9808 98.3708) (width 0.25) (layer "B.Cu") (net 2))
 (segment (start 150.024 98.386) (end 150.0392 98.3708) (width 0.25) (layer "B.Cu") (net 2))
 (segment (start 148.908 97.172) (end 148.908 97.27) (width 0.25) (layer "B.Cu") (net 2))
 (segment (start 148.908 97.27) (end 150.024 98.386) (width 0.25) (layer "B.Cu") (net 2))
 (segment (start 153.2156 96.1356) (end 152.1444 96.1356) (width 0.25) (layer "B.Cu") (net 2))
 (segment (start 150.9808 98.2235) (end 151.2334 97.9709) (width 0.25) (layer "B.Cu") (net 2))
 (segment (start 151.2334 97.9709) (end 151.2334 97.0466) (width 0.25) (layer "B.Cu") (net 2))
 (segment (start 150.9808 98.3708) (end 150.9808 98.2235) (width 0.25) (layer "B.Cu") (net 2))
 (segment (start 151.2334 97.0466) (end 151.58 96.7) (width 0.25) (layer "B.Cu") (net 2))
 (segment (start 148.908 97.27) (end 147.75 97.27) (width 0.25) (layer "B.Cu") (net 2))
 (segment (start 147.75 97.27) (end 147.18 96.7) (width 0.25) (layer "B.Cu") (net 2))
 (segment (start 149.41 99) (end 150.024 98.386) (width 0.25) (layer "B.Cu") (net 2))
 (segment (start 147.75 97.27) (end 147.75 103.15) (width 0.25) (layer "B.Cu") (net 2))
 (segment (start 150.9808 98.3708) (end 151.61 99) (width 0.25) (layer "B.Cu") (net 2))
 (segment (start 152.1444 96.1356) (end 151.58 96.7) (width 0.25) (layer "B.Cu") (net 2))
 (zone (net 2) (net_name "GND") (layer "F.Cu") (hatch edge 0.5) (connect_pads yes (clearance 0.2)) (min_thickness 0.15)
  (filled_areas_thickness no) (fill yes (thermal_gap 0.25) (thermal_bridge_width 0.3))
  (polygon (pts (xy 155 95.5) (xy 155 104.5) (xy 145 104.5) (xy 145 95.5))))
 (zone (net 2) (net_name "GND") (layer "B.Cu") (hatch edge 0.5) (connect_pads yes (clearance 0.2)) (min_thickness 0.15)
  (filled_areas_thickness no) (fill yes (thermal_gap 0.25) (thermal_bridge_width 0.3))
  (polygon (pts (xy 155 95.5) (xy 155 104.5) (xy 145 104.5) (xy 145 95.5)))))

